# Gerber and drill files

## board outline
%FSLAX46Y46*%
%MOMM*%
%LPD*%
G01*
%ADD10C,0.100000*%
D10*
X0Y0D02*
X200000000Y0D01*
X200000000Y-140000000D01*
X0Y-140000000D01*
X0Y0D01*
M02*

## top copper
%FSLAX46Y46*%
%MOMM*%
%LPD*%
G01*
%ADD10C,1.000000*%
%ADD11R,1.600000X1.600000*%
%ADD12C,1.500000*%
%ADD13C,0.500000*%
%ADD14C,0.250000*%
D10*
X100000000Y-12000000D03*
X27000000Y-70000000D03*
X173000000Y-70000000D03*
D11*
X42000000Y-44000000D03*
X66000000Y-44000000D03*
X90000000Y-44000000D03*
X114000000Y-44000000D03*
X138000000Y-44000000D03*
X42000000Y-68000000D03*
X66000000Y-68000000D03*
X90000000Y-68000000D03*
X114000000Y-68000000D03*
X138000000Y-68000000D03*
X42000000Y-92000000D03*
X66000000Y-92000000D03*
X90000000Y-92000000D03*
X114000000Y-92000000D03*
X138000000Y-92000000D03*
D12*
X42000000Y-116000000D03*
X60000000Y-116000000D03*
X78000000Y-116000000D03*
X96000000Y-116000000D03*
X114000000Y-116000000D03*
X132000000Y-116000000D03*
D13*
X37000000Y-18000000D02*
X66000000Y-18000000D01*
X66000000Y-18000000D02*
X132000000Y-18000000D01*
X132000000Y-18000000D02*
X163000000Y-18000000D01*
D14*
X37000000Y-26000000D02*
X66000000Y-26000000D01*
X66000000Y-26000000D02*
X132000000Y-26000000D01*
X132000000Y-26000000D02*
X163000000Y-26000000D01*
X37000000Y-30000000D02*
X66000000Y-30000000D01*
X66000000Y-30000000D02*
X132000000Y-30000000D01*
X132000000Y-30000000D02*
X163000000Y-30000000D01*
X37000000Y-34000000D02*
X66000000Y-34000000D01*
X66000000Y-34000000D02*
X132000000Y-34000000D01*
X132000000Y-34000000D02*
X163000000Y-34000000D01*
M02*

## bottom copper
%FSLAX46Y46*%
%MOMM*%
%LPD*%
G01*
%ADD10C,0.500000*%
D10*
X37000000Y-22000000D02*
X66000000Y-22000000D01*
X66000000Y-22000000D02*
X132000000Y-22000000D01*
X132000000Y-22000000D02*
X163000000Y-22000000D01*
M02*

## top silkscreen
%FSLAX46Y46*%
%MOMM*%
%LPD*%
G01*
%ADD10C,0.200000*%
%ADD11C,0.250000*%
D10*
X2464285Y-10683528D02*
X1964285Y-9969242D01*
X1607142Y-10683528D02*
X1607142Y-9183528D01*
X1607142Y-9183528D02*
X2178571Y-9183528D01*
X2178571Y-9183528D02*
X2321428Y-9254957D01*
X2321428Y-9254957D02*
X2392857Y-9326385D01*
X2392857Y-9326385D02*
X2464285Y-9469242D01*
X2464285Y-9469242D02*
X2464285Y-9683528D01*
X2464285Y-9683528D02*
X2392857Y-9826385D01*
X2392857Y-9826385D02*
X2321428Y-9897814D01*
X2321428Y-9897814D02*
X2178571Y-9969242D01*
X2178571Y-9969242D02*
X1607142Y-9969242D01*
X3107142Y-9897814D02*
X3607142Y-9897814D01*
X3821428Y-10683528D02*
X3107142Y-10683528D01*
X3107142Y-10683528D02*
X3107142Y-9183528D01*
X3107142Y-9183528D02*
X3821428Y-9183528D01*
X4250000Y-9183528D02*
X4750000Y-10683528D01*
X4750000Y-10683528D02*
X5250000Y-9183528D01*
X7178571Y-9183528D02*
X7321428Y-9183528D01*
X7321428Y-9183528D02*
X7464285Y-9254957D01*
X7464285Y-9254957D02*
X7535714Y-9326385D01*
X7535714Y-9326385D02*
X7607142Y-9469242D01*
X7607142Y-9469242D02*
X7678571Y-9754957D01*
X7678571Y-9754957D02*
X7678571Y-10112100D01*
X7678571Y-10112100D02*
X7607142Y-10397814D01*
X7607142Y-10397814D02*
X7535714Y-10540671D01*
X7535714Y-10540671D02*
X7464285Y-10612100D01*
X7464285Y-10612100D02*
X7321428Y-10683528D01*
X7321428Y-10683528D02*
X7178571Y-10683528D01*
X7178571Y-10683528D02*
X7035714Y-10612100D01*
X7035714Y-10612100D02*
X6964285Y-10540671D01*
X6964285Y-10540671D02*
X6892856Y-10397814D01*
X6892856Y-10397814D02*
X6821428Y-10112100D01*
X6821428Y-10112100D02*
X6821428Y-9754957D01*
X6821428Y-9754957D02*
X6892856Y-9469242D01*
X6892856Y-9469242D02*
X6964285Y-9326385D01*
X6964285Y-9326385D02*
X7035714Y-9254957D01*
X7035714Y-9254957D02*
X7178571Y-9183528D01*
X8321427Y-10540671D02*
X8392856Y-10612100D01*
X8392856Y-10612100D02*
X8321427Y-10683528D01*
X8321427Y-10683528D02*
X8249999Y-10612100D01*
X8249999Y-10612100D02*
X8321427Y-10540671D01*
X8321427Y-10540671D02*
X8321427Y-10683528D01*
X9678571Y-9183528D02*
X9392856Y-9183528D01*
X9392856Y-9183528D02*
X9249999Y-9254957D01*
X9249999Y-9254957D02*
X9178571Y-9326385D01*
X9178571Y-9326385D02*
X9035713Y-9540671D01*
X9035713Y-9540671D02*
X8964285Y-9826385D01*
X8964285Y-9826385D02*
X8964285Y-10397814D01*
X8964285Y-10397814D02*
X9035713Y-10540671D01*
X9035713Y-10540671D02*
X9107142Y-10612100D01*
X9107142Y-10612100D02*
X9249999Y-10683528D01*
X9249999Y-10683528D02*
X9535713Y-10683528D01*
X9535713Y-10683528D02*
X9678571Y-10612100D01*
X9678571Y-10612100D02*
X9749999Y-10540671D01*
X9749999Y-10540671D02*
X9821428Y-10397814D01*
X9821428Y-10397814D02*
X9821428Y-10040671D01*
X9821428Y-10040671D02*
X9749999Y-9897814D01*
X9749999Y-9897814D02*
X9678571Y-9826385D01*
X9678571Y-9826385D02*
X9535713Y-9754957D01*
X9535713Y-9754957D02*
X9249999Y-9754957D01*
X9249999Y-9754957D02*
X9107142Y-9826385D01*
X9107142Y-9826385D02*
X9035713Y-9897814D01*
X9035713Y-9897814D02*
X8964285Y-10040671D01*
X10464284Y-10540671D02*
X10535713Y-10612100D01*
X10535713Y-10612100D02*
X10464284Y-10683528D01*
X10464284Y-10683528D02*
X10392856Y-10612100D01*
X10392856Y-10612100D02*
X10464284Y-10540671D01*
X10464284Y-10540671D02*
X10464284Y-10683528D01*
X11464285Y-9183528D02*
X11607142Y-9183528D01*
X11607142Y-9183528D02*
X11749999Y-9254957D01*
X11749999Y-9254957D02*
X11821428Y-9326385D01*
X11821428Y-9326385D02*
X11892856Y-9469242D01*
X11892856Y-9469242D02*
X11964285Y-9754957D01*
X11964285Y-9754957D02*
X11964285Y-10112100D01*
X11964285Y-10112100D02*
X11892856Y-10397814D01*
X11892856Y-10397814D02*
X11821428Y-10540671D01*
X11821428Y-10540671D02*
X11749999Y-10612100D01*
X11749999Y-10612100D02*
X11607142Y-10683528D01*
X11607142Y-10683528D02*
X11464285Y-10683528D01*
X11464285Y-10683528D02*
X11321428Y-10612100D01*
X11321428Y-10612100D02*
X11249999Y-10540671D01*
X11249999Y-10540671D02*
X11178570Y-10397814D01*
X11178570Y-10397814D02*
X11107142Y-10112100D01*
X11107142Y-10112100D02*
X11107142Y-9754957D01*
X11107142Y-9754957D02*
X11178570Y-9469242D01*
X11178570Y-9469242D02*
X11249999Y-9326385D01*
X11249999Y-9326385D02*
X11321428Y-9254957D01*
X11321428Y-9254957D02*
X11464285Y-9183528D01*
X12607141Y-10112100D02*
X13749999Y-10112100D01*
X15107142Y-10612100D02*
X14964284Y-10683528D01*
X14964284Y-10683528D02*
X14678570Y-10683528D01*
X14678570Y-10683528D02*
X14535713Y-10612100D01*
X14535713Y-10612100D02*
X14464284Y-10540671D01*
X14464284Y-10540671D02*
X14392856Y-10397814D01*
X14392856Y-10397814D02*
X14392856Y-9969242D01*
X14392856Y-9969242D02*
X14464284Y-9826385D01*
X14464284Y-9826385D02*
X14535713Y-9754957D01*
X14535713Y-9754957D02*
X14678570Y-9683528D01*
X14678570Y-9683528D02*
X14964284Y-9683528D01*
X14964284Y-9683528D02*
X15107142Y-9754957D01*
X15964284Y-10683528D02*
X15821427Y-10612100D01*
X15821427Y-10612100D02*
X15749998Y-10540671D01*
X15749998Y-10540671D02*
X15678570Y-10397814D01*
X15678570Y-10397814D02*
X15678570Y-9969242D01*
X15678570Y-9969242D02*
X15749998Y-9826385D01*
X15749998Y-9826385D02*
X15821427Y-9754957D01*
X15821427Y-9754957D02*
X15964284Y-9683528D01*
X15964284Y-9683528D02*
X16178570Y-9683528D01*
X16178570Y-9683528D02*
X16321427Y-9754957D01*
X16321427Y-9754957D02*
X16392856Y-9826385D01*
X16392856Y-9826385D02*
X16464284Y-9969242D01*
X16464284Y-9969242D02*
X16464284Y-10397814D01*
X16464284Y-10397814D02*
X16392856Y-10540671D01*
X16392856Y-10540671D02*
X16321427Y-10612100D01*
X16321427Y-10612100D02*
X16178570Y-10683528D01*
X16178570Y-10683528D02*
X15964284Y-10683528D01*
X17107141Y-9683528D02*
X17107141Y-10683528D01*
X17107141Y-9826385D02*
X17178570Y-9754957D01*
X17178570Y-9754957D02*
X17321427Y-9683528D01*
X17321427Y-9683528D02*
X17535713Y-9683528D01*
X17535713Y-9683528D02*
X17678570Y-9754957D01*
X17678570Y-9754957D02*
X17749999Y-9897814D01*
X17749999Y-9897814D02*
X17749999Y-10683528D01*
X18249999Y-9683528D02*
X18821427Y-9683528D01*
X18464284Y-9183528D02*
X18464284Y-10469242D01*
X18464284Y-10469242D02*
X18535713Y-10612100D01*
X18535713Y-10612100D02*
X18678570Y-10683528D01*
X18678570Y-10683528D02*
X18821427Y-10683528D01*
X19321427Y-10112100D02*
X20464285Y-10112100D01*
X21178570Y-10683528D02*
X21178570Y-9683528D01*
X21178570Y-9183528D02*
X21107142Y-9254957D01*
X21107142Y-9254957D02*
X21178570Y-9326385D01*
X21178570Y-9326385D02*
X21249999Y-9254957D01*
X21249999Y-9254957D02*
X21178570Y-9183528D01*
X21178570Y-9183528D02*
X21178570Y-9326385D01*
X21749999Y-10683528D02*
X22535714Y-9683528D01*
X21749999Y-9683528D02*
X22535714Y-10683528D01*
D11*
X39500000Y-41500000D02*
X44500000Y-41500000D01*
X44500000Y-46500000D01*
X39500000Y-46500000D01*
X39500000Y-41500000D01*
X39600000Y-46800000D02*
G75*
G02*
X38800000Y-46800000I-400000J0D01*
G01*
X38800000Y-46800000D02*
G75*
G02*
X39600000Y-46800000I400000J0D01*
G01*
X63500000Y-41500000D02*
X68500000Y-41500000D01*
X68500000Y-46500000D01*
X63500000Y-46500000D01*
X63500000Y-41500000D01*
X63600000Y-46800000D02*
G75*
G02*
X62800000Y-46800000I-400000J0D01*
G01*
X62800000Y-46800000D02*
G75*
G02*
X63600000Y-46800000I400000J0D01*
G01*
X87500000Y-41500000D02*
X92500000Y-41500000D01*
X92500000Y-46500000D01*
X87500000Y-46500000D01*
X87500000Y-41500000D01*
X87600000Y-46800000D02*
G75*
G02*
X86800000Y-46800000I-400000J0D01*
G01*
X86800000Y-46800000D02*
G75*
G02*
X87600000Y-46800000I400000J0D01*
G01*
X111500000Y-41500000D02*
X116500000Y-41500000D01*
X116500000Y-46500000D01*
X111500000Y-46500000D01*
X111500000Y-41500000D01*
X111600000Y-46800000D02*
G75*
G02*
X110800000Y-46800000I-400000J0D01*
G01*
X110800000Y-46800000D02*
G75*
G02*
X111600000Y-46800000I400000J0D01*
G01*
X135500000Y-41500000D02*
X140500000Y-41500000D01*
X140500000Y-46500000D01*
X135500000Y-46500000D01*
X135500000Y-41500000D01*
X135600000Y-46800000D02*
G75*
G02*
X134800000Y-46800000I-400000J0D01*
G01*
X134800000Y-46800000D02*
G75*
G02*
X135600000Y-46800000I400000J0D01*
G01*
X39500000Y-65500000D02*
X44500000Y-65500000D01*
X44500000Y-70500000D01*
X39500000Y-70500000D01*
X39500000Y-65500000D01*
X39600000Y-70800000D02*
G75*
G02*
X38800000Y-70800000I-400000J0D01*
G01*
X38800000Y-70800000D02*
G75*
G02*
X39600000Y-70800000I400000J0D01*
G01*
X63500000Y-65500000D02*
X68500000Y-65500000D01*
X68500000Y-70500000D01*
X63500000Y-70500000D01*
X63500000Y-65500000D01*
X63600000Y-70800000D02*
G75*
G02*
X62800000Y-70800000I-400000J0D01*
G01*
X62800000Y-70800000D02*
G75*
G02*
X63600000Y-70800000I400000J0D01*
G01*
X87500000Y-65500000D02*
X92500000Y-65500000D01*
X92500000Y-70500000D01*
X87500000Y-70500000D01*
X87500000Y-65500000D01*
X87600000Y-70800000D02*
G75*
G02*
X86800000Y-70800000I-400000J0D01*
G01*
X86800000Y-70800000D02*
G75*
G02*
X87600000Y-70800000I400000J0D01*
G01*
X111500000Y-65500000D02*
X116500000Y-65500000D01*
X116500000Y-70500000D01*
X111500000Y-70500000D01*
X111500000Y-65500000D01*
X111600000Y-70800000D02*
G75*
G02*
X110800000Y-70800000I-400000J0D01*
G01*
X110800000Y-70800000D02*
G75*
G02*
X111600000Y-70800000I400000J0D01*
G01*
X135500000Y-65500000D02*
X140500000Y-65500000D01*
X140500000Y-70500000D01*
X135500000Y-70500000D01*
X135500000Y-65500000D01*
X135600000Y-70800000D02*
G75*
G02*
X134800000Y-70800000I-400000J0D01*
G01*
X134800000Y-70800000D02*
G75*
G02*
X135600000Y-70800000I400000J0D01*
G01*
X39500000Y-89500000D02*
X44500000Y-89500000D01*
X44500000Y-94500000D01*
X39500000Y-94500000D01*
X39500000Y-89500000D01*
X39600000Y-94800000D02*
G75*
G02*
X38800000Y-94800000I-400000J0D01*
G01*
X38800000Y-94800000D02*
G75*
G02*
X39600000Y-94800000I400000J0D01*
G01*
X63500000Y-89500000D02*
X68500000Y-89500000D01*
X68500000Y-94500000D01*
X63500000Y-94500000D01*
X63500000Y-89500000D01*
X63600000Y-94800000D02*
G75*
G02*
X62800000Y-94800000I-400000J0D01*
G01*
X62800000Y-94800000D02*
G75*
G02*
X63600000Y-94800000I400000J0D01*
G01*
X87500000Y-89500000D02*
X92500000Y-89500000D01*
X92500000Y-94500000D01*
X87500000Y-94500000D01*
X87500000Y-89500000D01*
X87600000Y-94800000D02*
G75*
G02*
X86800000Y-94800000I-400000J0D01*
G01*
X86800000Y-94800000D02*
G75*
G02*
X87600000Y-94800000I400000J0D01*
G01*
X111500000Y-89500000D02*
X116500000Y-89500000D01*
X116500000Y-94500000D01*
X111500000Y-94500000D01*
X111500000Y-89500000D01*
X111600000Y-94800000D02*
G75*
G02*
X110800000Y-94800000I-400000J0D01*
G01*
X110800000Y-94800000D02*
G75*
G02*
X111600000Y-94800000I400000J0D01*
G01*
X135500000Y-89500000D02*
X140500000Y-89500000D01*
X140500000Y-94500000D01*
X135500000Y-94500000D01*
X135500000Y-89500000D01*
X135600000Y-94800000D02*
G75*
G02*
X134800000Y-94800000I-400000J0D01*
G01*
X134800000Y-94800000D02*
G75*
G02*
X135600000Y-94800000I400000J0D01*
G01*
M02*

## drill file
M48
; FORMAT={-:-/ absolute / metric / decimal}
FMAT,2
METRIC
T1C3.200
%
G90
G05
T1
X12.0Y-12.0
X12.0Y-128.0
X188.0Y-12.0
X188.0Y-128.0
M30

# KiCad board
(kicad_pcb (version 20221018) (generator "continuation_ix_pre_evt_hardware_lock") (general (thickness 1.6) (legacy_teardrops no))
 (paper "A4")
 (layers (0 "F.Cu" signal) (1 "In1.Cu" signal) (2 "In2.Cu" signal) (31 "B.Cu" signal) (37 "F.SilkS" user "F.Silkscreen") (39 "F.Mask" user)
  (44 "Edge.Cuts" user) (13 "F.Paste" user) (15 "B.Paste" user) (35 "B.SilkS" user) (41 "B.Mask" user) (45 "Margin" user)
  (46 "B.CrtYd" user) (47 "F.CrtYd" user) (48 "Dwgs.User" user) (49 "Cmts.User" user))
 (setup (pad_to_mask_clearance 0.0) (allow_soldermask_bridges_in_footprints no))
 (gr_rect (start 0 0) (end 200.0 140.0) (stroke (width 0.1) (type default)) (fill none) (layer "Edge.Cuts"))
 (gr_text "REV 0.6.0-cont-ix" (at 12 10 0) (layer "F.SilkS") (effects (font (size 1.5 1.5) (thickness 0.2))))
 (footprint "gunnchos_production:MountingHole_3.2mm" (layer "F.Cu") (at 12.0 12.0)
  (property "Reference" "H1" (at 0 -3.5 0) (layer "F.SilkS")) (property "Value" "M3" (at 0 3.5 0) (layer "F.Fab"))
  (pad "" np_thru_hole circle (at 0 0) (size 3.2 3.2) (drill 3.2) (layers "*.Cu" "*.Mask")))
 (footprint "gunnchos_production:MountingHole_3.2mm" (layer "F.Cu") (at 188.0 12.0)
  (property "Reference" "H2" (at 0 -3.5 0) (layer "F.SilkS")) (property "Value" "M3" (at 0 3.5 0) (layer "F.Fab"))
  (pad "" np_thru_hole circle (at 0 0) (size 3.2 3.2) (drill 3.2) (layers "*.Cu" "*.Mask")))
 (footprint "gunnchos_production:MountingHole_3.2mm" (layer "F.Cu") (at 12.0 128.0)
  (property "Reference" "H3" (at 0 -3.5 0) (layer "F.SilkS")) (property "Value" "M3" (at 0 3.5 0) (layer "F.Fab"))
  (pad "" np_thru_hole circle (at 0 0) (size 3.2 3.2) (drill 3.2) (layers "*.Cu" "*.Mask")))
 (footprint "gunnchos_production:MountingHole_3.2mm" (layer "F.Cu") (at 188.0 128.0)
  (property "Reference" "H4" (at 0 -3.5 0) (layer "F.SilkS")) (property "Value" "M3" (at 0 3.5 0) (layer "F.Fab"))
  (pad "" np_thru_hole circle (at 0 0) (size 3.2 3.2) (drill 3.2) (layers "*.Cu" "*.Mask")))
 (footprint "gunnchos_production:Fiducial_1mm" (layer "F.Cu") (at 100.0 12.0)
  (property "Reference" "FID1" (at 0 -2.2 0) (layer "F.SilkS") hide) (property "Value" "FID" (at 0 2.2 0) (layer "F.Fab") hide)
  (pad "1" smd circle (at 0 0) (size 1 1) (layers "F.Cu") (solder_mask_margin 0.5)))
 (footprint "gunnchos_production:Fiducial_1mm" (layer "F.Cu") (at 27.0 70.0)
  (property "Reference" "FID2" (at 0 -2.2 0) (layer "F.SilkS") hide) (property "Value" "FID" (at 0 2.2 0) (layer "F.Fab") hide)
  (pad "1" smd circle (at 0 0) (size 1 1) (layers "F.Cu") (solder_mask_margin 0.5)))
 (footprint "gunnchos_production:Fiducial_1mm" (layer "F.Cu") (at 173.0 70.0)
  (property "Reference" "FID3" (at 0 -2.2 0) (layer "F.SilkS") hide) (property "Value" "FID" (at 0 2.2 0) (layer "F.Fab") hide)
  (pad "1" smd circle (at 0 0) (size 1 1) (layers "F.Cu") (solder_mask_margin 0.5)))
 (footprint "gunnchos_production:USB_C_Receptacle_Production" (layer "F.Cu") (at 42.00 44.00)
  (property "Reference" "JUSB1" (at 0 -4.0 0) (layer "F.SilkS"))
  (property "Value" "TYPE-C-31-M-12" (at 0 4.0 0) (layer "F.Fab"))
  (fp_rect (start -2.5 -2.5) (end 2.5 2.5) (layer "F.SilkS") (width 0.25) (fill none))
  (fp_circle (center -2.8 2.8) (end -2.4 2.8) (layer "F.SilkS") (width 0.25) (fill none))
  (pad "1" smd rect (at 0 0) (size 1.6 1.6) (layers "F.Cu" "F.Paste" "F.Mask")))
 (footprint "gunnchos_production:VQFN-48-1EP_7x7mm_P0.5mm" (layer "F.Cu") (at 66.00 44.00)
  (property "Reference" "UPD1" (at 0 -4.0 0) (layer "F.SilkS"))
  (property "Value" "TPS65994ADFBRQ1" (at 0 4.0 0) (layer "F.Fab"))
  (fp_rect (start -2.5 -2.5) (end 2.5 2.5) (layer "F.SilkS") (width 0.25) (fill none))
  (fp_circle (center -2.8 2.8) (end -2.4 2.8) (layer "F.SilkS") (width 0.25) (fill none))
  (pad "1" smd rect (at 0 0) (size 1.6 1.6) (layers "F.Cu" "F.Paste" "F.Mask")))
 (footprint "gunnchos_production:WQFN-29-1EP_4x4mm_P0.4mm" (layer "F.Cu") (at 90.00 44.00)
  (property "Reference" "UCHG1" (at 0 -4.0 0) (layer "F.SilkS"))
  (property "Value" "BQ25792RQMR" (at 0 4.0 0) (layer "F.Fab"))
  (fp_rect (start -2.5 -2.5) (end 2.5 2.5) (layer "F.SilkS") (width 0.25) (fill none))
  (fp_circle (center -2.8 2.8) (end -2.4 2.8) (layer "F.SilkS") (width 0.25) (fill none))
  (pad "1" smd rect (at 0 0) (size 1.6 1.6) (layers "F.Cu" "F.Paste" "F.Mask")))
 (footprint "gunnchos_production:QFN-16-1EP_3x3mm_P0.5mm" (layer "F.Cu") (at 114.00 44.00)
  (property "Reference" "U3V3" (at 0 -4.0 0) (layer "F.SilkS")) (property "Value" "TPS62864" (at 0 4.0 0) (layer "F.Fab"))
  (fp_rect (start -2.5 -2.5) (end 2.5 2.5) (layer "F.SilkS") (width 0.25) (fill none))
  (fp_circle (center -2.8 2.8) (end -2.4 2.8) (layer "F.SilkS") (width 0.25) (fill none))
  (pad "1" smd rect (at 0 0) (size 1.6 1.6) (layers "F.Cu" "F.Paste" "F.Mask")))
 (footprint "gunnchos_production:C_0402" (layer "F.Cu") (at 138.00 44.00) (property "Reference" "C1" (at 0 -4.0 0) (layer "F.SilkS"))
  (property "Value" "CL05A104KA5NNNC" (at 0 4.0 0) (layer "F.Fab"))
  (fp_rect (start -2.5 -2.5) (end 2.5 2.5) (layer "F.SilkS") (width 0.25) (fill none))
  (fp_circle (center -2.8 2.8) (end -2.4 2.8) (layer "F.SilkS") (width 0.25) (fill none))
  (pad "1" smd rect (at 0 0) (size 1.6 1.6) (layers "F.Cu" "F.Paste" "F.Mask")))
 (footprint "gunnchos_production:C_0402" (layer "F.Cu") (at 42.00 68.00) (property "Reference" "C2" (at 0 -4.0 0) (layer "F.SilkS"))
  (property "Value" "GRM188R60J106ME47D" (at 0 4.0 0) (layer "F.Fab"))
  (fp_rect (start -2.5 -2.5) (end 2.5 2.5) (layer "F.SilkS") (width 0.25) (fill none))
  (fp_circle (center -2.8 2.8) (end -2.4 2.8) (layer "F.SilkS") (width 0.25) (fill none))
  (pad "1" smd rect (at 0 0) (size 1.6 1.6) (layers "F.Cu" "F.Paste" "F.Mask")))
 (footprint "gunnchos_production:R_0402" (layer "F.Cu") (at 66.00 68.00) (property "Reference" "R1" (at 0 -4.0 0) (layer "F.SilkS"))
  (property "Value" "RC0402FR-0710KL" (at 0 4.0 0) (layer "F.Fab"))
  (fp_rect (start -2.5 -2.5) (end 2.5 2.5) (layer "F.SilkS") (width 0.25) (fill none))
  (fp_circle (center -2.8 2.8) (end -2.4 2.8) (layer "F.SilkS") (width 0.25) (fill none))
  (pad "1" smd rect (at 0 0) (size 1.6 1.6) (layers "F.Cu" "F.Paste" "F.Mask")))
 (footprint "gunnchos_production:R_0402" (layer "F.Cu") (at 90.00 68.00) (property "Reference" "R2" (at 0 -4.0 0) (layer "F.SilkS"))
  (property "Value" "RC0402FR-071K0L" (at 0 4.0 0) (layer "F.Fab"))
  (fp_rect (start -2.5 -2.5) (end 2.5 2.5) (layer "F.SilkS") (width 0.25) (fill none))
  (fp_circle (center -2.8 2.8) (end -2.4 2.8) (layer "F.SilkS") (width 0.25) (fill none))
  (pad "1" smd rect (at 0 0) (size 1.6 1.6) (layers "F.Cu" "F.Paste" "F.Mask")))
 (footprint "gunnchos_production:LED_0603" (layer "F.Cu") (at 114.00 68.00) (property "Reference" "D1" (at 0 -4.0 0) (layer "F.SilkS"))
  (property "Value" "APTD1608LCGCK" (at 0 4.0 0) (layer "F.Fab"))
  (fp_rect (start -2.5 -2.5) (end 2.5 2.5) (layer "F.SilkS") (width 0.25) (fill none))
  (fp_circle (center -2.8 2.8) (end -2.4 2.8) (layer "F.SilkS") (width 0.25) (fill none))
  (pad "1" smd rect (at 0 0) (size 1.6 1.6) (layers "F.Cu" "F.Paste" "F.Mask")))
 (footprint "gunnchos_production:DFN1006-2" (layer "F.Cu") (at 138.00 68.00)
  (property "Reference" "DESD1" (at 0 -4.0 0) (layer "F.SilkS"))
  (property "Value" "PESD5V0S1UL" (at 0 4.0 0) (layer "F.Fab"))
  (fp_rect (start -2.5 -2.5) (end 2.5 2.5) (layer "F.SilkS") (width 0.25) (fill none))
  (fp_circle (center -2.8 2.8) (end -2.4 2.8) (layer "F.SilkS") (width 0.25) (fill none))
  (pad "1" smd rect (at 0 0) (size 1.6 1.6) (layers "F.Cu" "F.Paste" "F.Mask")))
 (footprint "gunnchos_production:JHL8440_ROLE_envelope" (layer "F.Cu") (at 42.00 92.00)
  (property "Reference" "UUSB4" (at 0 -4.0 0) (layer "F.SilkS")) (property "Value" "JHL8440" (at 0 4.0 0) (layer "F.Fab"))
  (fp_rect (start -2.5 -2.5) (end 2.5 2.5) (layer "F.SilkS") (width 0.25) (fill none))
  (fp_circle (center -2.8 2.8) (end -2.4 2.8) (layer "F.SilkS") (width 0.25) (fill none))
  (pad "1" smd rect (at 0 0) (size 1.6 1.6) (layers "F.Cu" "F.Paste" "F.Mask")))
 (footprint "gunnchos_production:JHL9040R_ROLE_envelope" (layer "F.Cu") (at 66.00 92.00)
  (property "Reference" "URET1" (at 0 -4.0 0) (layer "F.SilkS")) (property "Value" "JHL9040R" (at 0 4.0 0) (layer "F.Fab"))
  (fp_rect (start -2.5 -2.5) (end 2.5 2.5) (layer "F.SilkS") (width 0.25) (fill none))
  (fp_circle (center -2.8 2.8) (end -2.4 2.8) (layer "F.SilkS") (width 0.25) (fill none))
  (pad "1" smd rect (at 0 0) (size 1.6 1.6) (layers "F.Cu" "F.Paste" "F.Mask")))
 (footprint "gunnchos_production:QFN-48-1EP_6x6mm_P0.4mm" (layer "F.Cu") (at 90.00 92.00)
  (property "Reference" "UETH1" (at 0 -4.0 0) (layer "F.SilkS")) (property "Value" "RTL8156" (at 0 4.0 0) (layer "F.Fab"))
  (fp_rect (start -2.5 -2.5) (end 2.5 2.5) (layer "F.SilkS") (width 0.25) (fill none))
  (fp_circle (center -2.8 2.8) (end -2.4 2.8) (layer "F.SilkS") (width 0.25) (fill none))
  (pad "1" smd rect (at 0 0) (size 1.6 1.6) (layers "F.Cu" "F.Paste" "F.Mask")))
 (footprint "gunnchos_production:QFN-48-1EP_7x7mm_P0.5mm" (layer "F.Cu") (at 114.00 92.00)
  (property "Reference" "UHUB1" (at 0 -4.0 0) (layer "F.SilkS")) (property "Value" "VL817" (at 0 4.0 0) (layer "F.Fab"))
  (fp_rect (start -2.5 -2.5) (end 2.5 2.5) (layer "F.SilkS") (width 0.25) (fill none))
  (fp_circle (center -2.8 2.8) (end -2.4 2.8) (layer "F.SilkS") (width 0.25) (fill none))
  (pad "1" smd rect (at 0 0) (size 1.6 1.6) (layers "F.Cu" "F.Paste" "F.Mask")))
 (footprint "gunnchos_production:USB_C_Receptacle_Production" (layer "F.Cu") (at 138.00 92.00)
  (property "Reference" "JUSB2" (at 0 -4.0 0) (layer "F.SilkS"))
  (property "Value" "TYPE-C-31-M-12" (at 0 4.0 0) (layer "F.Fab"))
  (fp_rect (start -2.5 -2.5) (end 2.5 2.5) (layer "F.SilkS") (width 0.25) (fill none))
  (fp_circle (center -2.8 2.8) (end -2.4 2.8) (layer "F.SilkS") (width 0.25) (fill none))
  (pad "1" smd rect (at 0 0) (size 1.6 1.6) (layers "F.Cu" "F.Paste" "F.Mask")))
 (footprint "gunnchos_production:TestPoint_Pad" (layer "F.Cu") (at 42.0 116.0) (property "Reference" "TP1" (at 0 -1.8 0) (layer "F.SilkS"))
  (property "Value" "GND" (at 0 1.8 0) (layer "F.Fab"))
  (pad "1" smd circle (at 0 0) (size 1.5 1.5) (layers "F.Cu" "F.Mask")))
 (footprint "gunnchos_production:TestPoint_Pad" (layer "F.Cu") (at 60.0 116.0) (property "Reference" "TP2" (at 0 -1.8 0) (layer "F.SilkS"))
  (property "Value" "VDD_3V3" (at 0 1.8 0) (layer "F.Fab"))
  (pad "1" smd circle (at 0 0) (size 1.5 1.5) (layers "F.Cu" "F.Mask")))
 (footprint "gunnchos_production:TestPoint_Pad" (layer "F.Cu") (at 78.0 116.0) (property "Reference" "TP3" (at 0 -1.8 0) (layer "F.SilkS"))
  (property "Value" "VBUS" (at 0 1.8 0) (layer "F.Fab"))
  (pad "1" smd circle (at 0 0) (size 1.5 1.5) (layers "F.Cu" "F.Mask")))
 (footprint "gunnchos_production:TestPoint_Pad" (layer "F.Cu") (at 96.0 116.0) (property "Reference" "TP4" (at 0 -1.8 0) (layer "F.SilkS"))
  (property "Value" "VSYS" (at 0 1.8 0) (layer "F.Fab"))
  (pad "1" smd circle (at 0 0) (size 1.5 1.5) (layers "F.Cu" "F.Mask")))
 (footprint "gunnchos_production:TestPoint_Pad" (layer "F.Cu") (at 114.0 116.0) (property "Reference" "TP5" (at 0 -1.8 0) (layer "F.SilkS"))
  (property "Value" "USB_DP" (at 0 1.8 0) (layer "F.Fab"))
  (pad "1" smd circle (at 0 0) (size 1.5 1.5) (layers "F.Cu" "F.Mask")))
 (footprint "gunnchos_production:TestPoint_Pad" (layer "F.Cu") (at 132.0 116.0) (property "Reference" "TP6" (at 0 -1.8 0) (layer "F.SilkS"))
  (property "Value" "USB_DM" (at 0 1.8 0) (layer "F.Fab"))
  (pad "1" smd circle (at 0 0) (size 1.5 1.5) (layers "F.Cu" "F.Mask")))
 (segment (start 37.00 18.00) (end 66.00 18.00) (width 0.5) (layer "F.Cu") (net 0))
 (segment (start 66.00 18.00) (end 132.00 18.00) (width 0.5) (layer "F.Cu") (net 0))
 (segment (start 132.00 18.00) (end 163.00 18.00) (width 0.5) (layer "F.Cu") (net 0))
 (segment (start 37.00 22.00) (end 66.00 22.00) (width 0.5) (layer "B.Cu") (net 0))
 (segment (start 66.00 22.00) (end 132.00 22.00) (width 0.5) (layer "B.Cu") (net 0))
 (segment (start 132.00 22.00) (end 163.00 22.00) (width 0.5) (layer "B.Cu") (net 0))
 (segment (start 37.00 26.00) (end 66.00 26.00) (width 0.25) (layer "F.Cu") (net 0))
 (segment (start 66.00 26.00) (end 132.00 26.00) (width 0.25) (layer "F.Cu") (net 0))
 (segment (start 132.00 26.00) (end 163.00 26.00) (width 0.25) (layer "F.Cu") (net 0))
 (segment (start 37.00 30.00) (end 66.00 30.00) (width 0.25) (layer "F.Cu") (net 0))
 (segment (start 66.00 30.00) (end 132.00 30.00) (width 0.25) (layer "F.Cu") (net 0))
 (segment (start 132.00 30.00) (end 163.00 30.00) (width 0.25) (layer "F.Cu") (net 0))
 (segment (start 37.00 34.00) (end 66.00 34.00) (width 0.25) (layer "F.Cu") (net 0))
 (segment (start 66.00 34.00) (end 132.00 34.00) (width 0.25) (layer "F.Cu") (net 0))
 (segment (start 132.00 34.00) (end 163.00 34.00) (width 0.25) (layer "F.Cu") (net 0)))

